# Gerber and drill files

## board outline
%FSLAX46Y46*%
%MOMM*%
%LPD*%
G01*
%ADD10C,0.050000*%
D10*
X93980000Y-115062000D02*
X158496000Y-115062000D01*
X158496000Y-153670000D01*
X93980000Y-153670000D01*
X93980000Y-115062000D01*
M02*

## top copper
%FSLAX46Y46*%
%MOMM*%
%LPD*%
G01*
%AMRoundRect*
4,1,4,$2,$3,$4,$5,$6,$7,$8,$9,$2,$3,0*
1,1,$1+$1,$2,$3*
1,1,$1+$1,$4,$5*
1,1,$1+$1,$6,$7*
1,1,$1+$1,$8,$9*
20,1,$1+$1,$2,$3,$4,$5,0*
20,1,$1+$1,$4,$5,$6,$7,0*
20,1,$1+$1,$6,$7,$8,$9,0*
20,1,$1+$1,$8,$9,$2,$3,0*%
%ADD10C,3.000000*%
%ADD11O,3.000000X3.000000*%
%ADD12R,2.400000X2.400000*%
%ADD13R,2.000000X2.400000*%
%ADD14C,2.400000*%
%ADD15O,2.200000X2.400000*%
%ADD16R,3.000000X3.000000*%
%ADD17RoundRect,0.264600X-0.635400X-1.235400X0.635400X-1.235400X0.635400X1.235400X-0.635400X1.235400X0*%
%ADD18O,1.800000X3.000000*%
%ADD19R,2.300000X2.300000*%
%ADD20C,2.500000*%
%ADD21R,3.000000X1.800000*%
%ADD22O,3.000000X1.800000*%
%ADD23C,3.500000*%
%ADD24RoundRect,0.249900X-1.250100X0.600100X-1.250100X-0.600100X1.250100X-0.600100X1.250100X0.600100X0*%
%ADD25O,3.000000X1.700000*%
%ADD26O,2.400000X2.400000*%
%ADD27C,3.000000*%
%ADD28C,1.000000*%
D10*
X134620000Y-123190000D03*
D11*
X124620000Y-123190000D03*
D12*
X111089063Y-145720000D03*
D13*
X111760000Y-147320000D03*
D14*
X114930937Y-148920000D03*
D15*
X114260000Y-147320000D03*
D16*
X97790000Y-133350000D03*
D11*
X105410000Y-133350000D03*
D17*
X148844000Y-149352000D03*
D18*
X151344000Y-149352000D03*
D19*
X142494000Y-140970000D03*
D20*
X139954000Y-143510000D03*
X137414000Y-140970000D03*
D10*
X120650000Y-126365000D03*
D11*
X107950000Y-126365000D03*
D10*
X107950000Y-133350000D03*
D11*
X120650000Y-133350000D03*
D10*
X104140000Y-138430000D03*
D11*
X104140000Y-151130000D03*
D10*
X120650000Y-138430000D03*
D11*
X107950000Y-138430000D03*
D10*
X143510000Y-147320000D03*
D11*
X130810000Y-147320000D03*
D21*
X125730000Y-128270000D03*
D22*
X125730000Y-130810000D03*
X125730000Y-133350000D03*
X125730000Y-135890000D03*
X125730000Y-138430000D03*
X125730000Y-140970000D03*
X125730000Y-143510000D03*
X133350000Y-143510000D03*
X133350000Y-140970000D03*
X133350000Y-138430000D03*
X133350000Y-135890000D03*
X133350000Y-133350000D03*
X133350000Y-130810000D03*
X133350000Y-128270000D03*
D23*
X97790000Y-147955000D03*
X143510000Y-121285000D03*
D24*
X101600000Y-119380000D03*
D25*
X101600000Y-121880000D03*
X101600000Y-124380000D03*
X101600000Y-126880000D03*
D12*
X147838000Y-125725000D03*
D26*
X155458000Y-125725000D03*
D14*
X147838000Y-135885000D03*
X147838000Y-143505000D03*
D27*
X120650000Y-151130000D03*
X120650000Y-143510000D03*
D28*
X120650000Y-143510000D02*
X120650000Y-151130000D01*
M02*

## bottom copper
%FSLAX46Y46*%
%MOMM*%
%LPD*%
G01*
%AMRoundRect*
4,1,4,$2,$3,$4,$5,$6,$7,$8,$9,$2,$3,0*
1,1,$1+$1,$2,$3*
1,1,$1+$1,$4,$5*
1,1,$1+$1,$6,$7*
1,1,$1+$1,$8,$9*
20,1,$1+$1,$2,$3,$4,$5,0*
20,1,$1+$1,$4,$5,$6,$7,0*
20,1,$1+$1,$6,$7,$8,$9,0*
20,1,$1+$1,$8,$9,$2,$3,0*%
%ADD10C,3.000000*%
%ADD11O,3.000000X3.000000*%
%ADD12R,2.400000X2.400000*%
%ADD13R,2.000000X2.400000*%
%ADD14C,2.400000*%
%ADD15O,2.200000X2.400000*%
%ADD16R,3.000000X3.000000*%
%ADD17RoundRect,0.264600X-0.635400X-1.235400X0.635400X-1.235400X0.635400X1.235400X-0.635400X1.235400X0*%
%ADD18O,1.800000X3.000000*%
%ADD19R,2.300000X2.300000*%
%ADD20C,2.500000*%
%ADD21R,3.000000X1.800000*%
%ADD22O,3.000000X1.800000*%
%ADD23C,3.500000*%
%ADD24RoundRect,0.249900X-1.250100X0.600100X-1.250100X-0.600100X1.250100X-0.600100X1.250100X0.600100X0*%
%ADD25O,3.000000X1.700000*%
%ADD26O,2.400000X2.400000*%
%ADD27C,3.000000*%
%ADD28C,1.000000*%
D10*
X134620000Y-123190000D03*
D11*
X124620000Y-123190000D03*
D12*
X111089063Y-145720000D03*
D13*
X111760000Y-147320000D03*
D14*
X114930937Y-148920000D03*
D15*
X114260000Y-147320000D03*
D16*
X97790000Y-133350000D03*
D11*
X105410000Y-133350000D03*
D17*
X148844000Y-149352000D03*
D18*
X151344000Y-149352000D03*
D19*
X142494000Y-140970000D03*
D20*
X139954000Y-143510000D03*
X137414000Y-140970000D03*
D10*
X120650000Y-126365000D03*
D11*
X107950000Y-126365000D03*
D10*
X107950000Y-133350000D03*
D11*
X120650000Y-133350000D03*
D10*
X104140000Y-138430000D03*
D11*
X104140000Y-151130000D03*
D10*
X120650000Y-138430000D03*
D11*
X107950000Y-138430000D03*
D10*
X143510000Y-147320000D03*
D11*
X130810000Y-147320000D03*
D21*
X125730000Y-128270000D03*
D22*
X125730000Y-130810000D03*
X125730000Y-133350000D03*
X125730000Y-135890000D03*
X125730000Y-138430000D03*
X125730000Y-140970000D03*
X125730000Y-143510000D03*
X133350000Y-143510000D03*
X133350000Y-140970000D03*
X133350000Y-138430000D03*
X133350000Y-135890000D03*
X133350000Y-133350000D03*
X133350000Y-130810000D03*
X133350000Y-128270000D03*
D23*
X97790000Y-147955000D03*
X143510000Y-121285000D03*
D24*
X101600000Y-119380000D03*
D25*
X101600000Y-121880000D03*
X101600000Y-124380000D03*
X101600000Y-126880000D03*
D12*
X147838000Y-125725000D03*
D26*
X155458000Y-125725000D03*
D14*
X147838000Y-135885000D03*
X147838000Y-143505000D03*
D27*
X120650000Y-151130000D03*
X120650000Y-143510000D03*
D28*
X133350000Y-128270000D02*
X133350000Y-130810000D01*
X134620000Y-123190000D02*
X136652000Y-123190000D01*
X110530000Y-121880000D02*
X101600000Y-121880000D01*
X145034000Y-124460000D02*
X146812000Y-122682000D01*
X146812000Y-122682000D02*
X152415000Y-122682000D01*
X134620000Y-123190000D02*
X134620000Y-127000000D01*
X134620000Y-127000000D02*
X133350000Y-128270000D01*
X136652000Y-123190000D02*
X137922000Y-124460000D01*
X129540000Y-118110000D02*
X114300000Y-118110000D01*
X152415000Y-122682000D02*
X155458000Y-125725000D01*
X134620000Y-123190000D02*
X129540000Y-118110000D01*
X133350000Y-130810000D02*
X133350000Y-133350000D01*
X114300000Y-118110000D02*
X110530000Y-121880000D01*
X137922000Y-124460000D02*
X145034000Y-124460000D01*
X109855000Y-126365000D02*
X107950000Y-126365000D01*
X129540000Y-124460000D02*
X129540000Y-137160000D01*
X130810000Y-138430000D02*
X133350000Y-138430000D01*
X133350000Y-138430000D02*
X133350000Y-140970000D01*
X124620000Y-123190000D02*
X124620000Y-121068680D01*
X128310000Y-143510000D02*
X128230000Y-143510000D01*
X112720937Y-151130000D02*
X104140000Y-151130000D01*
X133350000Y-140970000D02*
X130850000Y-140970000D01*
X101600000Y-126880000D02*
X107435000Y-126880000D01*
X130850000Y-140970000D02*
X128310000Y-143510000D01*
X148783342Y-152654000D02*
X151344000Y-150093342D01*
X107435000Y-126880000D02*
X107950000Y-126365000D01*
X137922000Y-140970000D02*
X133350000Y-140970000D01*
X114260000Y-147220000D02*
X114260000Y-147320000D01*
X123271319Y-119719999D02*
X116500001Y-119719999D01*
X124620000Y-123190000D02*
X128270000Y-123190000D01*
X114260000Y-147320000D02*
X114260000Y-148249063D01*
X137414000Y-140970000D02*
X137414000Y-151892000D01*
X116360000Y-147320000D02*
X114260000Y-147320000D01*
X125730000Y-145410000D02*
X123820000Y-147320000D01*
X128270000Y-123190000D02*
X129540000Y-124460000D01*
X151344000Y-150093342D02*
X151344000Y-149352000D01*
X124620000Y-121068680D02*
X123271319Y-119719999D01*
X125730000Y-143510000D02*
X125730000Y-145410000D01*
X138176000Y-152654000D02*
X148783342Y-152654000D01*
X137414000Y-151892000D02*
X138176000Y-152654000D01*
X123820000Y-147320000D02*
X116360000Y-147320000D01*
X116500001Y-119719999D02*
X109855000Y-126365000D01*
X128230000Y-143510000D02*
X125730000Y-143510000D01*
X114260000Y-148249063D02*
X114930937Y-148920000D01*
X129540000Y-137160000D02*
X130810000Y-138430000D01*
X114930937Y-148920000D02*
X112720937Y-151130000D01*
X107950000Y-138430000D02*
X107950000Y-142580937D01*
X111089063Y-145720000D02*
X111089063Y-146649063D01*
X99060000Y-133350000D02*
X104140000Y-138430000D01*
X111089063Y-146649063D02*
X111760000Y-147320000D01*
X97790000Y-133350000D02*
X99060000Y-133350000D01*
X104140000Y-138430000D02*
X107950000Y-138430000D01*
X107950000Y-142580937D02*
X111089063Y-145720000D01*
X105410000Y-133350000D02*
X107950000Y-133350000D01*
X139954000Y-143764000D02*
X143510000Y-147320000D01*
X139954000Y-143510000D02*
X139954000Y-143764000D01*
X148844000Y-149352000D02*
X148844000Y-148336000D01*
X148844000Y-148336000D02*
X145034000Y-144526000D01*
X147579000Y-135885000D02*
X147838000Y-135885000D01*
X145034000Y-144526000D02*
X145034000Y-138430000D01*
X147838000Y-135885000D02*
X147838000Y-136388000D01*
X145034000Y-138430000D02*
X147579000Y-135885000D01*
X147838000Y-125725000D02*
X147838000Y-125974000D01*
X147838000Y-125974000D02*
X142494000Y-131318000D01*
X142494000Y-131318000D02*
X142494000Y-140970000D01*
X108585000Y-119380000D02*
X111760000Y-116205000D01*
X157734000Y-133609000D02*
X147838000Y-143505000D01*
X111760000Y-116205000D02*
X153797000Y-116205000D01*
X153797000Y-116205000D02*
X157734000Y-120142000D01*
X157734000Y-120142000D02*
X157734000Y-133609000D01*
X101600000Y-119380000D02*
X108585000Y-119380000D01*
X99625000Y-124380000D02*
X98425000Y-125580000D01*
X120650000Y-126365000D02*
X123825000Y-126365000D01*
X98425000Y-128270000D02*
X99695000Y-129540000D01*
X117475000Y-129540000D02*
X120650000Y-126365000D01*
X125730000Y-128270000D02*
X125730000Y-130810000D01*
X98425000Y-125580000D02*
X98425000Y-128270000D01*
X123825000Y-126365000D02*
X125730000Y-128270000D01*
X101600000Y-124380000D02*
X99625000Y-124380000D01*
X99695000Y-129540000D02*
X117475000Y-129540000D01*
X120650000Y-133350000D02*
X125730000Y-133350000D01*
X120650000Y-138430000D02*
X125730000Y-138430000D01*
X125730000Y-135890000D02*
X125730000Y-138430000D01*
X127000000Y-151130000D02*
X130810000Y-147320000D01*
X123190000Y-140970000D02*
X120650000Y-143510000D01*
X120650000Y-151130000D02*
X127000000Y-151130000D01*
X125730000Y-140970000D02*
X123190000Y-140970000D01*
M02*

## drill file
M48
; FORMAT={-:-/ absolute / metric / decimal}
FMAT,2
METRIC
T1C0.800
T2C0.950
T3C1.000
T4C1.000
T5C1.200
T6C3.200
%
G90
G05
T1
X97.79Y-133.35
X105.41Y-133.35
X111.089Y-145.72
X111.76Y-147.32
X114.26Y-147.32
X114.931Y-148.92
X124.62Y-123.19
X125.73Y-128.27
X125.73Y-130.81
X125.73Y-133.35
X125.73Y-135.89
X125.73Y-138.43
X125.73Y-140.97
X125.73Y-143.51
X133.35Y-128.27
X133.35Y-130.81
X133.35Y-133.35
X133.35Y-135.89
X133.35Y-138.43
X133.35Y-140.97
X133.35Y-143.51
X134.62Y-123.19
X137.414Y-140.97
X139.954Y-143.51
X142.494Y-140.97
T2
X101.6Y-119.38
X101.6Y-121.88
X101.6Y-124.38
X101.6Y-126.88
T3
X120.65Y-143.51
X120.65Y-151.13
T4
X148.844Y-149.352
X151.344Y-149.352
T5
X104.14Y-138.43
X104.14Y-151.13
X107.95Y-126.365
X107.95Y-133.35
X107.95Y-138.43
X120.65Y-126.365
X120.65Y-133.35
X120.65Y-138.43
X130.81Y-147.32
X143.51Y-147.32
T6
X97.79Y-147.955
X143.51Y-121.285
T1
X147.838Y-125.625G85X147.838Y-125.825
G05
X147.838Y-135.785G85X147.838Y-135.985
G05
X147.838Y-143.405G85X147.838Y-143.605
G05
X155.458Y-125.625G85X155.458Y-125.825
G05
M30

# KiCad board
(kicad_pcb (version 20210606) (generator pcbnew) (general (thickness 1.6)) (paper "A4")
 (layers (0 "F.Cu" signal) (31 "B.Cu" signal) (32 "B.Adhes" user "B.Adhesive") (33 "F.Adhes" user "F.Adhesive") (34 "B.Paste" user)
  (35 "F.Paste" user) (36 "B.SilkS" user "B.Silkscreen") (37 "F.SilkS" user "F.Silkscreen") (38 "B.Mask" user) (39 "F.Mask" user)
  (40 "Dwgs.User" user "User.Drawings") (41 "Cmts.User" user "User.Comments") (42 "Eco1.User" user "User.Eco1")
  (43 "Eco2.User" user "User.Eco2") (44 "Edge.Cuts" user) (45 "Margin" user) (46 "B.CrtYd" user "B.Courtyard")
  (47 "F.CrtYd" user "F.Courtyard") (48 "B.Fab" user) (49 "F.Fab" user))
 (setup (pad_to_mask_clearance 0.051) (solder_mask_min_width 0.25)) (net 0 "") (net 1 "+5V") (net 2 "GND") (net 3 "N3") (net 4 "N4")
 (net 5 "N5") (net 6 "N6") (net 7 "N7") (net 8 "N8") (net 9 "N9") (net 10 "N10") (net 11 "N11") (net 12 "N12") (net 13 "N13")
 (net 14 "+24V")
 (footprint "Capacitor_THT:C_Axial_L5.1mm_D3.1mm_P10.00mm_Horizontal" (layer "F.Cu") (at 134.62 123.19 180)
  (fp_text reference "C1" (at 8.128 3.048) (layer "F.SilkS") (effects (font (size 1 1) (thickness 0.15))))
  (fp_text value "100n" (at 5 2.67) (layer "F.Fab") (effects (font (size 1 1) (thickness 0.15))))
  (pad "1" thru_hole circle locked (at 0 0 180) (size 3 3) (drill 0.8) (layers *.Cu *.Mask) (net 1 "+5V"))
  (pad "2" thru_hole oval locked (at 10 0 180) (size 3 3) (drill 0.8) (layers *.Cu *.Mask) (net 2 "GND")))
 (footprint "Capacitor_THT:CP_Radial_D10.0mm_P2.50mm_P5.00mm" (layer "F.Cu") (at 111.76 147.32)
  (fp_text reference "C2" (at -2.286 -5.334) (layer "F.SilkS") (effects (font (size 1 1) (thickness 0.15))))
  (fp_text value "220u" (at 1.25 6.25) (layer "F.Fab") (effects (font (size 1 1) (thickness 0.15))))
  (pad "1" thru_hole rect locked (at -0.670937 -1.6) (size 2.4 2.4) (drill 0.8) (layers *.Cu *.Mask) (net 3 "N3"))
  (pad "1" thru_hole rect locked (at 0 0) (size 2 2.4) (drill 0.8) (layers *.Cu *.Mask) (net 3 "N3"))
  (pad "2" thru_hole circle locked (at 3.170937 1.6) (size 2.4 2.4) (drill 0.8) (layers *.Cu *.Mask) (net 2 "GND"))
  (pad "2" thru_hole oval locked (at 2.5 0) (size 2.2 2.4) (drill 0.8) (layers *.Cu *.Mask) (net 2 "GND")))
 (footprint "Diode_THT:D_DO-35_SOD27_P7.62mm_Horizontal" (layer "F.Cu") (at 97.79 133.35)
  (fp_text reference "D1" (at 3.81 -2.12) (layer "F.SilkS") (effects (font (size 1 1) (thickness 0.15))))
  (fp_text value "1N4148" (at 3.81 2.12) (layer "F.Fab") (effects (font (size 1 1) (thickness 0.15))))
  (pad "1" thru_hole rect locked (at 0 0) (size 3 3) (drill 0.8) (layers *.Cu *.Mask) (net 3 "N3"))
  (pad "2" thru_hole oval locked (at 7.62 0) (size 3 3) (drill 0.8) (layers *.Cu *.Mask) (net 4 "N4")))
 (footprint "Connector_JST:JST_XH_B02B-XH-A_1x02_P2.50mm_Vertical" (layer "F.Cu") (at 148.844 149.352)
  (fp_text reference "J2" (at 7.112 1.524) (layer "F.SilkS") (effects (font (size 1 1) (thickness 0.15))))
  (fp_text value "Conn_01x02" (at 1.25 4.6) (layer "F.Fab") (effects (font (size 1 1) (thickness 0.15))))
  (pad "1" thru_hole roundrect locked (at 0 0) (size 1.8 3) (drill 1) (layers *.Cu *.Mask) (roundrect_rratio 0.147) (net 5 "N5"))
  (pad "2" thru_hole oval locked (at 2.5 0) (size 1.8 3) (drill 1) (layers *.Cu *.Mask) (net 2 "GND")))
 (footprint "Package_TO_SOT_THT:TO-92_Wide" (layer "F.Cu") (at 142.494 140.97 180)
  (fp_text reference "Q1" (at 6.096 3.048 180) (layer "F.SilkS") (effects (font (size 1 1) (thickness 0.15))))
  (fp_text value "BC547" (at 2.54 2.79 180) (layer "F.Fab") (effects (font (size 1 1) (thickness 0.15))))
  (pad "1" thru_hole rect locked (at 0 0 270) (size 2.3 2.3) (drill 0.8) (layers *.Cu *.Mask) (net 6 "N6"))
  (pad "2" thru_hole circle locked (at 2.54 -2.54 270) (size 2.5 2.5) (drill 0.8) (layers *.Cu *.Mask) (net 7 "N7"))
  (pad "3" thru_hole circle locked (at 5.08 0 180) (size 2.5 2.5) (drill 0.8) (layers *.Cu *.Mask) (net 2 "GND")))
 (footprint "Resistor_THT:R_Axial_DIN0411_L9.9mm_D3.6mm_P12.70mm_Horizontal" (layer "F.Cu") (at 120.65 126.365 180)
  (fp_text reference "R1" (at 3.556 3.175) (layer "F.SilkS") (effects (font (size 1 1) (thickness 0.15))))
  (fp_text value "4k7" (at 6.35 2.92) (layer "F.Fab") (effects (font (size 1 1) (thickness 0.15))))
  (pad "1" thru_hole circle locked (at 0 0 180) (size 3 3) (drill 1.2) (layers *.Cu *.Mask) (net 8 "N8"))
  (pad "2" thru_hole oval locked (at 12.7 0 180) (size 3 3) (drill 1.2) (layers *.Cu *.Mask) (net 2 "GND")))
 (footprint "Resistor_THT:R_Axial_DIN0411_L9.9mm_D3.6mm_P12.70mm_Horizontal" (layer "F.Cu") (at 107.95 133.35)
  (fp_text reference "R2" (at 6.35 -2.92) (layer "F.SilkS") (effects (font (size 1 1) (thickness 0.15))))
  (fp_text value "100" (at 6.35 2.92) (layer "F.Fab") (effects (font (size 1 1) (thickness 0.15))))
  (pad "1" thru_hole circle locked (at 0 0) (size 3 3) (drill 1.2) (layers *.Cu *.Mask) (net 4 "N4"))
  (pad "2" thru_hole oval locked (at 12.7 0) (size 3 3) (drill 1.2) (layers *.Cu *.Mask) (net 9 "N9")))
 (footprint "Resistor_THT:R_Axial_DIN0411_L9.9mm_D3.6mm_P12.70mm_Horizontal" (layer "F.Cu") (at 104.14 138.43 -90)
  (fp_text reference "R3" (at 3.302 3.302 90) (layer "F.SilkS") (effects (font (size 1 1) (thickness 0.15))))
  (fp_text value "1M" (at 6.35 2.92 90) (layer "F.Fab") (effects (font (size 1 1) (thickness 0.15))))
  (pad "1" thru_hole circle locked (at 0 0 270) (size 3 3) (drill 1.2) (layers *.Cu *.Mask) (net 3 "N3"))
  (pad "2" thru_hole oval locked (at 12.7 0 270) (size 3 3) (drill 1.2) (layers *.Cu *.Mask) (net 2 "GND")))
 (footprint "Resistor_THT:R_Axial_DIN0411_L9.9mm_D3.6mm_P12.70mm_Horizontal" (layer "F.Cu") (at 120.65 138.43 180)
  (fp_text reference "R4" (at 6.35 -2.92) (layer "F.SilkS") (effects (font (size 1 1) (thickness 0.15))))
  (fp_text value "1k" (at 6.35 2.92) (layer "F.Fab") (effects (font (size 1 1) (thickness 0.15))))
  (pad "1" thru_hole circle locked (at 0 0 180) (size 3 3) (drill 1.2) (layers *.Cu *.Mask) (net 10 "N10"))
  (pad "2" thru_hole oval locked (at 12.7 0 180) (size 3 3) (drill 1.2) (layers *.Cu *.Mask) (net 3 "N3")))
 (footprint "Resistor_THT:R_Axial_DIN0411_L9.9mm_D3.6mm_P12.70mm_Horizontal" (layer "F.Cu") (at 143.51 147.32 180)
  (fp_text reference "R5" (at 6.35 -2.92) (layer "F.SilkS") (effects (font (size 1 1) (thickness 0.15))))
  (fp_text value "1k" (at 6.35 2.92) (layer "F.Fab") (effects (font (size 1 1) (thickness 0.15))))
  (pad "1" thru_hole circle locked (at 0 0 180) (size 3 3) (drill 1.2) (layers *.Cu *.Mask) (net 7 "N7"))
  (pad "2" thru_hole oval locked (at 12.7 0 180) (size 3 3) (drill 1.2) (layers *.Cu *.Mask) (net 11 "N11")))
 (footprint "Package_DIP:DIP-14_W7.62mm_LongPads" (layer "F.Cu") (at 125.73 128.27)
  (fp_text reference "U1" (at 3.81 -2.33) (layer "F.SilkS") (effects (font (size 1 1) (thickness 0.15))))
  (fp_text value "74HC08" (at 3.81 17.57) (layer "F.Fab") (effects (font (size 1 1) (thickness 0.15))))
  (pad "1" thru_hole rect locked (at 0 0) (size 3 1.8) (drill 0.8) (layers *.Cu *.Mask) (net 8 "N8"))
  (pad "2" thru_hole oval locked (at 0 2.54) (size 3 1.8) (drill 0.8) (layers *.Cu *.Mask) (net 8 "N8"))
  (pad "3" thru_hole oval locked (at 0 5.08) (size 3 1.8) (drill 0.8) (layers *.Cu *.Mask) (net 9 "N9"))
  (pad "4" thru_hole oval locked (at 0 7.62) (size 3 1.8) (drill 0.8) (layers *.Cu *.Mask) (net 10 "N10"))
  (pad "5" thru_hole oval locked (at 0 10.16) (size 3 1.8) (drill 0.8) (layers *.Cu *.Mask) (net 10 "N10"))
  (pad "6" thru_hole oval locked (at 0 12.7) (size 3 1.8) (drill 0.8) (layers *.Cu *.Mask) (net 11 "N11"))
  (pad "7" thru_hole oval locked (at 0 15.24) (size 3 1.8) (drill 0.8) (layers *.Cu *.Mask) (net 2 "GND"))
  (pad "8" thru_hole oval locked (at 7.62 15.24) (size 3 1.8) (drill 0.8) (layers *.Cu *.Mask) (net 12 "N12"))
  (pad "9" thru_hole oval locked (at 7.62 12.7) (size 3 1.8) (drill 0.8) (layers *.Cu *.Mask) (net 2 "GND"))
  (pad "10" thru_hole oval locked (at 7.62 10.16) (size 3 1.8) (drill 0.8) (layers *.Cu *.Mask) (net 2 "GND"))
  (pad "11" thru_hole oval locked (at 7.62 7.62) (size 3 1.8) (drill 0.8) (layers *.Cu *.Mask) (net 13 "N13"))
  (pad "12" thru_hole oval locked (at 7.62 5.08) (size 3 1.8) (drill 0.8) (layers *.Cu *.Mask) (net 1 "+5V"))
  (pad "13" thru_hole oval locked (at 7.62 2.54) (size 3 1.8) (drill 0.8) (layers *.Cu *.Mask) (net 1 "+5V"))
  (pad "14" thru_hole oval locked (at 7.62 0) (size 3 1.8) (drill 0.8) (layers *.Cu *.Mask) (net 1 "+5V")))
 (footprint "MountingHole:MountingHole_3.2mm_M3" (layer "F.Cu") (at 97.79 147.955)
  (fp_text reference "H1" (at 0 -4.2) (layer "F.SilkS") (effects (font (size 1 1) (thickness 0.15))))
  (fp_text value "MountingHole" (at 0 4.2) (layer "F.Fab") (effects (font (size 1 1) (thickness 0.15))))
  (pad "" np_thru_hole circle locked (at 0 0) (size 3.5 3.5) (drill 3.2) (layers *.Cu *.Mask)))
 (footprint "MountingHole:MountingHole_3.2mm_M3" (layer "F.Cu") (at 143.51 121.285)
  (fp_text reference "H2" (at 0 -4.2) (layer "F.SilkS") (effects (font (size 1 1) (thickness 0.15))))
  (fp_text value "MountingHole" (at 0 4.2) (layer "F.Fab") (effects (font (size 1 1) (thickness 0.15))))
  (pad "" np_thru_hole circle locked (at 0 0) (size 3.5 3.5) (drill 3.2) (layers *.Cu *.Mask)))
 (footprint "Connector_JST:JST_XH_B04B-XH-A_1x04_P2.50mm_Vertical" (layer "F.Cu") (at 101.6 119.38 -90)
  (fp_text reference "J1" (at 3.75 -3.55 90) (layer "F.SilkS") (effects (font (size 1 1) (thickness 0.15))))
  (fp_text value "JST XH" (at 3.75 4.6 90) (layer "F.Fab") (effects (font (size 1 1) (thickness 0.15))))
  (pad "1" thru_hole roundrect locked (at 0 0 270) (size 1.7 3) (drill 0.95) (layers *.Cu *.Mask) (roundrect_rratio 0.147) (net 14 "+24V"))
  (pad "2" thru_hole oval locked (at 2.5 0 270) (size 1.7 3) (drill 0.95) (layers *.Cu *.Mask) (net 1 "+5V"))
  (pad "3" thru_hole oval locked (at 5 0 270) (size 1.7 3) (drill 0.95) (layers *.Cu *.Mask) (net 8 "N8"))
  (pad "4" thru_hole oval locked (at 7.5 0 270) (size 1.7 3) (drill 0.95) (layers *.Cu *.Mask) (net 2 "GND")))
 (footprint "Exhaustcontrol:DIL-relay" (layer "F.Cu") (at 147.838 125.725)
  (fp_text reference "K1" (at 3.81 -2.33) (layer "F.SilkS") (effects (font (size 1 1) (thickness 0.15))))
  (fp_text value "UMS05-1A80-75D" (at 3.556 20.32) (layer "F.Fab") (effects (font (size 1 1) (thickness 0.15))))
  (pad "1" thru_hole rect locked (at 0 0) (size 2.4 2.4) (drill oval 0.8 1) (layers *.Cu *.Mask) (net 6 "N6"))
  (pad "2" thru_hole oval locked (at 7.62 0) (size 2.4 2.4) (drill oval 0.8 1) (layers *.Cu *.Mask) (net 1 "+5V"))
  (pad "3" thru_hole circle locked (at 0 10.16) (size 2.4 2.4) (drill oval 0.8 1) (layers *.Cu *.Mask) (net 5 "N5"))
  (pad "4" thru_hole circle locked (at 0 17.78) (size 2.4 2.4) (drill oval 0.8 1) (layers *.Cu *.Mask) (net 14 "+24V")))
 (gr_rect (start 93.98 115.062) (end 158.496 153.67) (layer "Edge.Cuts") (width 0.05) (fill none))
 (segment (start 133.35 128.27) (end 133.35 130.81) (width 1) (layer "B.Cu") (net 1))
 (segment (start 134.62 123.19) (end 136.652 123.19) (width 1) (layer "B.Cu") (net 1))
 (segment (start 110.53 121.88) (end 101.6 121.88) (width 1) (layer "B.Cu") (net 1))
 (segment (start 145.034 124.46) (end 146.812 122.682) (width 1) (layer "B.Cu") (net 1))
 (segment (start 146.812 122.682) (end 152.415 122.682) (width 1) (layer "B.Cu") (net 1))
 (segment (start 134.62 123.19) (end 134.62 127) (width 1) (layer "B.Cu") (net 1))
 (segment (start 134.62 127) (end 133.35 128.27) (width 1) (layer "B.Cu") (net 1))
 (segment (start 136.652 123.19) (end 137.922 124.46) (width 1) (layer "B.Cu") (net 1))
 (segment (start 129.54 118.11) (end 114.3 118.11) (width 1) (layer "B.Cu") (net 1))
 (segment (start 152.415 122.682) (end 155.458 125.725) (width 1) (layer "B.Cu") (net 1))
 (segment (start 134.62 123.19) (end 129.54 118.11) (width 1) (layer "B.Cu") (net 1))
 (segment (start 133.35 130.81) (end 133.35 133.35) (width 1) (layer "B.Cu") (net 1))
 (segment (start 114.3 118.11) (end 110.53 121.88) (width 1) (layer "B.Cu") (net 1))
 (segment (start 137.922 124.46) (end 145.034 124.46) (width 1) (layer "B.Cu") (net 1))
 (segment (start 109.855 126.365) (end 107.95 126.365) (width 1) (layer "B.Cu") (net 2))
 (segment (start 129.54 124.46) (end 129.54 137.16) (width 1) (layer "B.Cu") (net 2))
 (segment (start 130.81 138.43) (end 133.35 138.43) (width 1) (layer "B.Cu") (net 2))
 (segment (start 133.35 138.43) (end 133.35 140.97) (width 1) (layer "B.Cu") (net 2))
 (segment (start 124.62 123.19) (end 124.62 121.06868) (width 1) (layer "B.Cu") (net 2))
 (segment (start 128.31 143.51) (end 128.23 143.51) (width 1) (layer "B.Cu") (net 2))
 (segment (start 112.720937 151.13) (end 104.14 151.13) (width 1) (layer "B.Cu") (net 2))
 (segment (start 133.35 140.97) (end 130.85 140.97) (width 1) (layer "B.Cu") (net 2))
 (segment (start 101.6 126.88) (end 107.435 126.88) (width 1) (layer "B.Cu") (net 2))
 (segment (start 130.85 140.97) (end 128.31 143.51) (width 1) (layer "B.Cu") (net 2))
 (segment (start 148.783342 152.654) (end 151.344 150.093342) (width 1) (layer "B.Cu") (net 2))
 (segment (start 107.435 126.88) (end 107.95 126.365) (width 1) (layer "B.Cu") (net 2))
 (segment (start 137.922 140.97) (end 133.35 140.97) (width 1) (layer "B.Cu") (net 2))
 (segment (start 114.26 147.22) (end 114.26 147.32) (width 1) (layer "B.Cu") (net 2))
 (segment (start 123.271319 119.719999) (end 116.500001 119.719999) (width 1) (layer "B.Cu") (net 2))
 (segment (start 124.62 123.19) (end 128.27 123.19) (width 1) (layer "B.Cu") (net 2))
 (segment (start 114.26 147.32) (end 114.26 148.249063) (width 1) (layer "B.Cu") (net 2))
 (segment (start 137.414 140.97) (end 137.414 151.892) (width 1) (layer "B.Cu") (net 2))
 (segment (start 116.36 147.32) (end 114.26 147.32) (width 1) (layer "B.Cu") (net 2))
 (segment (start 125.73 145.41) (end 123.82 147.32) (width 1) (layer "B.Cu") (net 2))
 (segment (start 128.27 123.19) (end 129.54 124.46) (width 1) (layer "B.Cu") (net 2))
 (segment (start 151.344 150.093342) (end 151.344 149.352) (width 1) (layer "B.Cu") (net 2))
 (segment (start 124.62 121.06868) (end 123.271319 119.719999) (width 1) (layer "B.Cu") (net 2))
 (segment (start 125.73 143.51) (end 125.73 145.41) (width 1) (layer "B.Cu") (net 2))
 (segment (start 138.176 152.654) (end 148.783342 152.654) (width 1) (layer "B.Cu") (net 2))
 (segment (start 137.414 151.892) (end 138.176 152.654) (width 1) (layer "B.Cu") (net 2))
 (segment (start 123.82 147.32) (end 116.36 147.32) (width 1) (layer "B.Cu") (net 2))
 (segment (start 116.500001 119.719999) (end 109.855 126.365) (width 1) (layer "B.Cu") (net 2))
 (segment (start 128.23 143.51) (end 125.73 143.51) (width 1) (layer "B.Cu") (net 2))
 (segment (start 114.26 148.249063) (end 114.930937 148.92) (width 1) (layer "B.Cu") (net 2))
 (segment (start 129.54 137.16) (end 130.81 138.43) (width 1) (layer "B.Cu") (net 2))
 (segment (start 114.930937 148.92) (end 112.720937 151.13) (width 1) (layer "B.Cu") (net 2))
 (segment (start 107.95 138.43) (end 107.95 142.580937) (width 1) (layer "B.Cu") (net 3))
 (segment (start 111.089063 145.72) (end 111.089063 146.649063) (width 1) (layer "B.Cu") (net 3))
 (segment (start 99.06 133.35) (end 104.14 138.43) (width 1) (layer "B.Cu") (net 3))
 (segment (start 111.089063 146.649063) (end 111.76 147.32) (width 1) (layer "B.Cu") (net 3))
 (segment (start 97.79 133.35) (end 99.06 133.35) (width 1) (layer "B.Cu") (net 3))
 (segment (start 104.14 138.43) (end 107.95 138.43) (width 1) (layer "B.Cu") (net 3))
 (segment (start 107.95 142.580937) (end 111.089063 145.72) (width 1) (layer "B.Cu") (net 3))
 (segment (start 105.41 133.35) (end 107.95 133.35) (width 1) (layer "B.Cu") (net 4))
 (segment (start 139.954 143.764) (end 143.51 147.32) (width 1) (layer "B.Cu") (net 7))
 (segment (start 139.954 143.51) (end 139.954 143.764) (width 1) (layer "B.Cu") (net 7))
 (segment (start 148.844 149.352) (end 148.844 148.336) (width 1) (layer "B.Cu") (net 5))
 (segment (start 148.844 148.336) (end 145.034 144.526) (width 1) (layer "B.Cu") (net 5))
 (segment (start 147.579 135.885) (end 147.838 135.885) (width 1) (layer "B.Cu") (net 5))
 (segment (start 145.034 144.526) (end 145.034 138.43) (width 1) (layer "B.Cu") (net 5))
 (segment (start 147.838 135.885) (end 147.838 136.388) (width 1) (layer "B.Cu") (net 5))
 (segment (start 145.034 138.43) (end 147.579 135.885) (width 1) (layer "B.Cu") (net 5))
 (segment (start 147.838 125.725) (end 147.838 125.974) (width 1) (layer "B.Cu") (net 6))
 (segment (start 147.838 125.974) (end 142.494 131.318) (width 1) (layer "B.Cu") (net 6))
 (segment (start 142.494 131.318) (end 142.494 140.97) (width 1) (layer "B.Cu") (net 6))
 (segment (start 108.585 119.38) (end 111.76 116.205) (width 1) (layer "B.Cu") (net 14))
 (segment (start 157.734 133.609) (end 147.838 143.505) (width 1) (layer "B.Cu") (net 14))
 (segment (start 111.76 116.205) (end 153.797 116.205) (width 1) (layer "B.Cu") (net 14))
 (segment (start 153.797 116.205) (end 157.734 120.142) (width 1) (layer "B.Cu") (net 14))
 (segment (start 157.734 120.142) (end 157.734 133.609) (width 1) (layer "B.Cu") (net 14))
 (segment (start 101.6 119.38) (end 108.585 119.38) (width 1) (layer "B.Cu") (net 14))
 (segment (start 99.625 124.38) (end 98.425 125.58) (width 1) (layer "B.Cu") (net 8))
 (segment (start 120.65 126.365) (end 123.825 126.365) (width 1) (layer "B.Cu") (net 8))
 (segment (start 98.425 128.27) (end 99.695 129.54) (width 1) (layer "B.Cu") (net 8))
 (segment (start 117.475 129.54) (end 120.65 126.365) (width 1) (layer "B.Cu") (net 8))
 (segment (start 125.73 128.27) (end 125.73 130.81) (width 1) (layer "B.Cu") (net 8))
 (segment (start 98.425 125.58) (end 98.425 128.27) (width 1) (layer "B.Cu") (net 8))
 (segment (start 123.825 126.365) (end 125.73 128.27) (width 1) (layer "B.Cu") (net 8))
 (segment (start 101.6 124.38) (end 99.625 124.38) (width 1) (layer "B.Cu") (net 8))
 (segment (start 99.695 129.54) (end 117.475 129.54) (width 1) (layer "B.Cu") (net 8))
 (segment (start 120.65 133.35) (end 125.73 133.35) (width 1) (layer "B.Cu") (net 9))
 (segment (start 120.65 138.43) (end 125.73 138.43) (width 1) (layer "B.Cu") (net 10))
 (segment (start 125.73 135.89) (end 125.73 138.43) (width 1) (layer "B.Cu") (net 10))
 (segment (start 120.65 143.51) (end 120.65 151.13) (width 1) (layer "F.Cu") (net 11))
 (via (at 120.65 151.13) (size 3) (drill 1) (layers "F.Cu" "B.Cu") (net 11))
 (via (at 120.65 143.51) (size 3) (drill 1) (layers "F.Cu" "B.Cu") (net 11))
 (segment (start 127 151.13) (end 130.81 147.32) (width 1) (layer "B.Cu") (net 11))
 (segment (start 123.19 140.97) (end 120.65 143.51) (width 1) (layer "B.Cu") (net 11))
 (segment (start 120.65 151.13) (end 127 151.13) (width 1) (layer "B.Cu") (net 11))
 (segment (start 125.73 140.97) (end 123.19 140.97) (width 1) (layer "B.Cu") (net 11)))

